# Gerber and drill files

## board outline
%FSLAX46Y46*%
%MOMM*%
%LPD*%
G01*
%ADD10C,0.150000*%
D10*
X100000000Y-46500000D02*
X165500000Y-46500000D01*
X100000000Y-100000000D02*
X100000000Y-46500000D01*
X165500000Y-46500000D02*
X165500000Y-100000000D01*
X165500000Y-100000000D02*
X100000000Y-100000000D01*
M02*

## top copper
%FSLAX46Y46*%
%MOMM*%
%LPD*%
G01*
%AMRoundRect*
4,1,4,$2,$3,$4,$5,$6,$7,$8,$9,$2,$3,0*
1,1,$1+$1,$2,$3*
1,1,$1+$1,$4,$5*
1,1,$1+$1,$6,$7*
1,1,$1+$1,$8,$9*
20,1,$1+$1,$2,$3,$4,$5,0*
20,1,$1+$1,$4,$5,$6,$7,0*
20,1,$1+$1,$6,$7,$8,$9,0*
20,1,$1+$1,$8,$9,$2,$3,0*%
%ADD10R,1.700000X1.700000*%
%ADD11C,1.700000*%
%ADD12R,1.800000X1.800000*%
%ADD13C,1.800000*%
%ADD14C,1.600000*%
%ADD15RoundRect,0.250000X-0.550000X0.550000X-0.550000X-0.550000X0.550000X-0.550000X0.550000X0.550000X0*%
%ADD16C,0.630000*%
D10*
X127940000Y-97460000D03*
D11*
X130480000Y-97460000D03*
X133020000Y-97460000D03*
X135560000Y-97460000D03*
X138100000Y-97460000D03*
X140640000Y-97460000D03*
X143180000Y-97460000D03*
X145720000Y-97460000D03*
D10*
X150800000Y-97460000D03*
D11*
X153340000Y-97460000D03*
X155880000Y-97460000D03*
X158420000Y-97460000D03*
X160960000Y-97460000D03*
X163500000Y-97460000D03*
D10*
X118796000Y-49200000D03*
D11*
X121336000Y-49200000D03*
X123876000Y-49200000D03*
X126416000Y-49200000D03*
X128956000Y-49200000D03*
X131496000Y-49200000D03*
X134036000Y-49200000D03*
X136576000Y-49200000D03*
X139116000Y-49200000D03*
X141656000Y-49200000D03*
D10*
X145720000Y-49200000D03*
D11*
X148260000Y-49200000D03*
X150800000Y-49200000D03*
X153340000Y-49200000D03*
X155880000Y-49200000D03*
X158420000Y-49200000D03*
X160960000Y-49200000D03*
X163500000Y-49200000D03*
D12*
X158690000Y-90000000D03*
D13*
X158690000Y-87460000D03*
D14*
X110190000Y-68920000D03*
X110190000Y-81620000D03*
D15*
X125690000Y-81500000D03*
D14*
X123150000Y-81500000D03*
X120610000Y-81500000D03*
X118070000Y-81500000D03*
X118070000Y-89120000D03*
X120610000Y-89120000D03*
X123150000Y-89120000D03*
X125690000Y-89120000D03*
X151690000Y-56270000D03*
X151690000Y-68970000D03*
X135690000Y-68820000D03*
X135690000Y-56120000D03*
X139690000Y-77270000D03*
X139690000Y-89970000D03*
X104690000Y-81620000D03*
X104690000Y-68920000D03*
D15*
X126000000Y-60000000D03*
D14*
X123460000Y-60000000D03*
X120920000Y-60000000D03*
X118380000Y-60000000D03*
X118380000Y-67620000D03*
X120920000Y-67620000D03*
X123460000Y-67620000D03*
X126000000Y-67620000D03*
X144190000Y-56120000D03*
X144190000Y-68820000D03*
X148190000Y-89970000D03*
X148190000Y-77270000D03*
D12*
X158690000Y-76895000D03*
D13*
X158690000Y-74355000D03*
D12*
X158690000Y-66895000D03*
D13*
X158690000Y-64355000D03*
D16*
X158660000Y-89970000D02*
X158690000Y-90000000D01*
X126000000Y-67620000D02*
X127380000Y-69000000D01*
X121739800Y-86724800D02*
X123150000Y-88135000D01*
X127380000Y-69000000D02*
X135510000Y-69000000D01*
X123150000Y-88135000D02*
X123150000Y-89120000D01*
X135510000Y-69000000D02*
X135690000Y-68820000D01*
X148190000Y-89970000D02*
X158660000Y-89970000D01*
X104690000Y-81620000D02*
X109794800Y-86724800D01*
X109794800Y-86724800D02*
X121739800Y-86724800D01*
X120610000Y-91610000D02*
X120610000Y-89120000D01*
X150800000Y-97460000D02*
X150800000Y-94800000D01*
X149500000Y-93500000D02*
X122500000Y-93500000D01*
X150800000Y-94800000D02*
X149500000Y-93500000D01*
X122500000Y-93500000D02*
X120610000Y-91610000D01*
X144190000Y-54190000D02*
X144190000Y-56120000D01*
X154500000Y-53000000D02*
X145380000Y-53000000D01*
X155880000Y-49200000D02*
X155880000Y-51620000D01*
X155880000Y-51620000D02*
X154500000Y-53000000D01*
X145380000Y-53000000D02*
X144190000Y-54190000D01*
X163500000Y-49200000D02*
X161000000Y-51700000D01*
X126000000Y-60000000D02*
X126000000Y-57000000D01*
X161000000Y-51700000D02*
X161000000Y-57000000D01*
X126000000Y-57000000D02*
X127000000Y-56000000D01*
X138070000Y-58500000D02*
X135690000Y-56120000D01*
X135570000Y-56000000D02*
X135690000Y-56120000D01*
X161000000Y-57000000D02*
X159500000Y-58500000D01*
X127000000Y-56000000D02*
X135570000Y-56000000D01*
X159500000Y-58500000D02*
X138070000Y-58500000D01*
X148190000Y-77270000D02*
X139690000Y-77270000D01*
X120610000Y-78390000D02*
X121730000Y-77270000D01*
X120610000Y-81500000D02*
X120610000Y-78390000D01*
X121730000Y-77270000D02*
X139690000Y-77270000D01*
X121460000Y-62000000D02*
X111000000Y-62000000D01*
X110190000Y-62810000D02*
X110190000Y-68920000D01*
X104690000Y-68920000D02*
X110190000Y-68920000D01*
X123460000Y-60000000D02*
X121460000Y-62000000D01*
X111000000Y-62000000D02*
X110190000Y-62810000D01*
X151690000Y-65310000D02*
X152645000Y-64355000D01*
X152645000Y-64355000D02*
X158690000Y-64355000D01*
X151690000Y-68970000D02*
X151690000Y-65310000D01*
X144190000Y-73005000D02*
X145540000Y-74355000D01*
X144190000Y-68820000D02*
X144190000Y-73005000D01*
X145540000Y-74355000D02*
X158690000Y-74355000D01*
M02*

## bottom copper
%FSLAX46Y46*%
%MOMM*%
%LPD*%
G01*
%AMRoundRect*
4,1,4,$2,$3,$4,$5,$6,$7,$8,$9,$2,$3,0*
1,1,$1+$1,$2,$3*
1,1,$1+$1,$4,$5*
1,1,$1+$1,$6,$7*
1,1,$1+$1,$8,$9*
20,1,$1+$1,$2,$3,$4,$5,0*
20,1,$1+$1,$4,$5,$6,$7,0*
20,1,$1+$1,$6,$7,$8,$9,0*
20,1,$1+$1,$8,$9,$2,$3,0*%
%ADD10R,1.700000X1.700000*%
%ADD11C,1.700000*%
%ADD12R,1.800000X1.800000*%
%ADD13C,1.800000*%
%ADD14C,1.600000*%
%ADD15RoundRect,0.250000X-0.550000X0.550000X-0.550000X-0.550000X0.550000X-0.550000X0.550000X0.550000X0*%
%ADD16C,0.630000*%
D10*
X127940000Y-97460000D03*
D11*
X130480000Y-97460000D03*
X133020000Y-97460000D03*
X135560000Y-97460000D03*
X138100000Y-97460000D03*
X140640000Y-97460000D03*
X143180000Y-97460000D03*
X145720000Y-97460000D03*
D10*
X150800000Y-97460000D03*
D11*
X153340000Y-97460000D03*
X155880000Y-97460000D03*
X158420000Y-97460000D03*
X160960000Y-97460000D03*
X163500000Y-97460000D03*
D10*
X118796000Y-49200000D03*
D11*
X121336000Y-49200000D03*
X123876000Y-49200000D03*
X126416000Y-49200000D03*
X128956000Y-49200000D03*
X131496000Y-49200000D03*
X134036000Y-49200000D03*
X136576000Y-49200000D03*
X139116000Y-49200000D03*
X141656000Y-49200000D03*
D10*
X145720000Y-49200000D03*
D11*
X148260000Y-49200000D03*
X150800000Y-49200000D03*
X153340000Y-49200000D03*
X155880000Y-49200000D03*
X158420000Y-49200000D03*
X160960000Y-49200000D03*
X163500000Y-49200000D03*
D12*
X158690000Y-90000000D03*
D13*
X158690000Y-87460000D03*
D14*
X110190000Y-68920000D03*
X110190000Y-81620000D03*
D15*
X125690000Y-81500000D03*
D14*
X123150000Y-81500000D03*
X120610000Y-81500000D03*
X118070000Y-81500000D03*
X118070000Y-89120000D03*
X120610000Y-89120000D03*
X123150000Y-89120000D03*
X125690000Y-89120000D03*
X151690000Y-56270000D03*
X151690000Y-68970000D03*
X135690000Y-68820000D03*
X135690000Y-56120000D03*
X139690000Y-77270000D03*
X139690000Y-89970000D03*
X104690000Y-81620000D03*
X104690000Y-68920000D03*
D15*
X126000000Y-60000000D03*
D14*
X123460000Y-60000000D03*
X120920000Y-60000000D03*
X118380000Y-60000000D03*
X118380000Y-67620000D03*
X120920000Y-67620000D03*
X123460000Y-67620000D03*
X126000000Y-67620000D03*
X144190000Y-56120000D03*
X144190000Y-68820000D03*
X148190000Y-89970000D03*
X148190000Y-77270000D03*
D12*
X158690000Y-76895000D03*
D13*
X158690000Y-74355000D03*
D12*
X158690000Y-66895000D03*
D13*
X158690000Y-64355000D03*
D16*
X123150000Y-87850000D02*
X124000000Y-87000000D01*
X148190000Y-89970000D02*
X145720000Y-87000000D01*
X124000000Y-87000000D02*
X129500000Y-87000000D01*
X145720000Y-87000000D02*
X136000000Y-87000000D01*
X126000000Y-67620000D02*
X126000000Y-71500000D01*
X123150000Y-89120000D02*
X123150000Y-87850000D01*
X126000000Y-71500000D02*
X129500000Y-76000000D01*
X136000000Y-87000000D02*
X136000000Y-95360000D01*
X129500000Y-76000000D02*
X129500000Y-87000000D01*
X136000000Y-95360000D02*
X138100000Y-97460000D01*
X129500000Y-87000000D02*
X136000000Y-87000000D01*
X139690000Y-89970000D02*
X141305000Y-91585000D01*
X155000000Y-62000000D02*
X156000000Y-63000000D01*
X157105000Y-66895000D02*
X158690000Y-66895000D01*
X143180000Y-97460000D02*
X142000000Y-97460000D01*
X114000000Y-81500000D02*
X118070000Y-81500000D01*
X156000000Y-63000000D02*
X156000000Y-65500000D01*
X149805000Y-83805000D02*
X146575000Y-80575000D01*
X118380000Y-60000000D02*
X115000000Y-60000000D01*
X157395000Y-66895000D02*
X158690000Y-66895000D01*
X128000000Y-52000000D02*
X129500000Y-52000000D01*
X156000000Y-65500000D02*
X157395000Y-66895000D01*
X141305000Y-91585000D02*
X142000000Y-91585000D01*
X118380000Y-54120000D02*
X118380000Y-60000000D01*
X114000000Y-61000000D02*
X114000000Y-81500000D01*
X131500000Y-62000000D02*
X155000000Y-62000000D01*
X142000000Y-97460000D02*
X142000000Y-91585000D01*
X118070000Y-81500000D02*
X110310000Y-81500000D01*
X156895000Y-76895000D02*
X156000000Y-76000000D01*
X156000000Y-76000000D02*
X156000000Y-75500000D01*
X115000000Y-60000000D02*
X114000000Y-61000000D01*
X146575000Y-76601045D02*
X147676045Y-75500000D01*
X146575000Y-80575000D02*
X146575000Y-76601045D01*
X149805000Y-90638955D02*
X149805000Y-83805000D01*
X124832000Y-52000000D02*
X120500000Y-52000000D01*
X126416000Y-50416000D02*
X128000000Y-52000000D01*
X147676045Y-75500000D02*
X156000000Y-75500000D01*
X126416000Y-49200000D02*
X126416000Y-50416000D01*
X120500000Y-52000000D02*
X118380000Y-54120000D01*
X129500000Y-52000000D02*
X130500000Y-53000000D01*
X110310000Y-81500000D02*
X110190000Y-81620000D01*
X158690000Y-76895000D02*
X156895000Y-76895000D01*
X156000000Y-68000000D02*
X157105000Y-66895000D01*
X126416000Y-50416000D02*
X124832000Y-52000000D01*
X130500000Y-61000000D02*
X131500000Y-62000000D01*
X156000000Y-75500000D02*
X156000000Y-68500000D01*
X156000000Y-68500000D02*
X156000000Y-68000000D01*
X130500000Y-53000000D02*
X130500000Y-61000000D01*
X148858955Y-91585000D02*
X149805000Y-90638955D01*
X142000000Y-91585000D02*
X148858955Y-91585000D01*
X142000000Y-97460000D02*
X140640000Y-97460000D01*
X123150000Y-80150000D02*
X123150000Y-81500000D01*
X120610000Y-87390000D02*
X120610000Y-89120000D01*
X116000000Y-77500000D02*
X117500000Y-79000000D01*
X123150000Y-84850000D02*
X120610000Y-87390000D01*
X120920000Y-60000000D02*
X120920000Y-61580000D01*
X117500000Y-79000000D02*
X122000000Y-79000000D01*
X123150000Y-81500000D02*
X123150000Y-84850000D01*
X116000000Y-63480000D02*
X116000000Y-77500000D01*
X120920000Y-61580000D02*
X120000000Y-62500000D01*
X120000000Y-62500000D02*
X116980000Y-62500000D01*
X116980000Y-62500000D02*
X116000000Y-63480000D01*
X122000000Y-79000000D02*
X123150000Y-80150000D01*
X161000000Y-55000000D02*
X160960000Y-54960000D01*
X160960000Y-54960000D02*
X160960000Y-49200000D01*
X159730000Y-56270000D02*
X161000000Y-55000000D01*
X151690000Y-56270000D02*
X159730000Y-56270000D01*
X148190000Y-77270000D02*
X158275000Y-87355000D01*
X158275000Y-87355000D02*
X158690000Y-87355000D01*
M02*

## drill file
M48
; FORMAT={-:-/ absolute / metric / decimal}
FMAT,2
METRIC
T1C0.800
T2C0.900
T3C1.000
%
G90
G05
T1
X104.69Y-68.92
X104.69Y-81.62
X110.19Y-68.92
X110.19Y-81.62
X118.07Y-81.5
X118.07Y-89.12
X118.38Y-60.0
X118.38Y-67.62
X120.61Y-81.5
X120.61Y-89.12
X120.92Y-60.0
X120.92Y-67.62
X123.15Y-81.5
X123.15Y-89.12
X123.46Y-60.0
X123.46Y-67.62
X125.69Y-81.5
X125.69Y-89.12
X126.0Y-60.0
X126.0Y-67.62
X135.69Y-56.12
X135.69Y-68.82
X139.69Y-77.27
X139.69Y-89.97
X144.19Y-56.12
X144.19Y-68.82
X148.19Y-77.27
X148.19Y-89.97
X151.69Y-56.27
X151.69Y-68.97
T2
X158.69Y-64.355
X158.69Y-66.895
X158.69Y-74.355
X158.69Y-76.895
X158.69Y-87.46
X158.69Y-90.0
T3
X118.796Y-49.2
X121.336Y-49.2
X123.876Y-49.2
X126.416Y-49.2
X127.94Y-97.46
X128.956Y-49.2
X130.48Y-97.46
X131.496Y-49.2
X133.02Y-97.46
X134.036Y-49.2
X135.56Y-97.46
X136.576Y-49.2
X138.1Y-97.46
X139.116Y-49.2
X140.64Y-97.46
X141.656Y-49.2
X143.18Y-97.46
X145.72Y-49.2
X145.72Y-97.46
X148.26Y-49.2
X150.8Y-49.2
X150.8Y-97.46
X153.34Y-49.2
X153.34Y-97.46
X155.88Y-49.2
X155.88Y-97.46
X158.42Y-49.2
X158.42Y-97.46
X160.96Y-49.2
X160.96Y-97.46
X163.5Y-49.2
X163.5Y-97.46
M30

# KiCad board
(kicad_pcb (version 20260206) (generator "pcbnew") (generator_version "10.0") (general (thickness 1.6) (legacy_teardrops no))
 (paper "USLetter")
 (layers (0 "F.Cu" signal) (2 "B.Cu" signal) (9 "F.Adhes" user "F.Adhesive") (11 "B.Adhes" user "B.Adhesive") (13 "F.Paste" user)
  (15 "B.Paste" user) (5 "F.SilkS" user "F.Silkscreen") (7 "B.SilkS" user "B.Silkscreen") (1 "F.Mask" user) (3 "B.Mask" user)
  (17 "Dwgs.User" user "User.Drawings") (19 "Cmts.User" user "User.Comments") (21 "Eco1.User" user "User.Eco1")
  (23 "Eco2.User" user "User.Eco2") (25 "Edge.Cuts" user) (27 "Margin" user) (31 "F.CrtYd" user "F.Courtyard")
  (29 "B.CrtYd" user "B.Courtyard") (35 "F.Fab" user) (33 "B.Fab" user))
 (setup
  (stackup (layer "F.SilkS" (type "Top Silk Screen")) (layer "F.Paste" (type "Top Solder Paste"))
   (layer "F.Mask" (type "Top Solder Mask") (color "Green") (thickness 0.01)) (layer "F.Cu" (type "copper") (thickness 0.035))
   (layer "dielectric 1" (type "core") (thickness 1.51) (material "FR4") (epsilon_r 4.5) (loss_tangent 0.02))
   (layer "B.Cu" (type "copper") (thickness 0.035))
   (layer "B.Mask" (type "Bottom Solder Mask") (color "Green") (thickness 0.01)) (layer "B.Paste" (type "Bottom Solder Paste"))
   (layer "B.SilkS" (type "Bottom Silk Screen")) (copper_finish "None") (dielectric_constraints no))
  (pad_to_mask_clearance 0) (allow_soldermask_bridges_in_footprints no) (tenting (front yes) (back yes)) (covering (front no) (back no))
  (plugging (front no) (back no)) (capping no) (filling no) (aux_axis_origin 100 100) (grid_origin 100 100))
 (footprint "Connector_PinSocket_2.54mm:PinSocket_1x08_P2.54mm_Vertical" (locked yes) (layer "F.Cu") (at 127.94 97.46 90)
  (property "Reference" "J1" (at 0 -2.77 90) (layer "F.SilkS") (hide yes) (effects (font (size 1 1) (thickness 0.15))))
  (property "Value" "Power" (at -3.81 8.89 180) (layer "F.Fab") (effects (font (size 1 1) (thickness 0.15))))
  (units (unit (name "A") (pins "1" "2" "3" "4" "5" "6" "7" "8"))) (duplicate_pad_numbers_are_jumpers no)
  (pad "1" thru_hole rect (at 0 0 90) (size 1.7 1.7) (drill 1) (layers "*.Cu" "*.Mask") (remove_unused_layers no)
   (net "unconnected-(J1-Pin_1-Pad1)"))
  (pad "2" thru_hole circle (at 0 2.54 90) (size 1.7 1.7) (drill 1) (layers "*.Cu" "*.Mask") (remove_unused_layers no) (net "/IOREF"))
  (pad "3" thru_hole circle (at 0 5.08 90) (size 1.7 1.7) (drill 1) (layers "*.Cu" "*.Mask") (remove_unused_layers no) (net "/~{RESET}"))
  (pad "4" thru_hole circle (at 0 7.62 90) (size 1.7 1.7) (drill 1) (layers "*.Cu" "*.Mask") (remove_unused_layers no) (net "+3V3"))
  (pad "5" thru_hole circle (at 0 10.16 90) (size 1.7 1.7) (drill 1) (layers "*.Cu" "*.Mask") (remove_unused_layers no) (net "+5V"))
  (pad "6" thru_hole circle (at 0 12.7 90) (size 1.7 1.7) (drill 1) (layers "*.Cu" "*.Mask") (remove_unused_layers no) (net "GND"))
  (pad "7" thru_hole circle (at 0 15.24 90) (size 1.7 1.7) (drill 1) (layers "*.Cu" "*.Mask") (remove_unused_layers no) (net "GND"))
  (pad "8" thru_hole circle (at 0 17.78 90) (size 1.7 1.7) (drill 1) (layers "*.Cu" "*.Mask") (remove_unused_layers no) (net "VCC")))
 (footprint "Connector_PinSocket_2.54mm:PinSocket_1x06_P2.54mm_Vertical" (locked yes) (layer "F.Cu") (at 150.8 97.46 90)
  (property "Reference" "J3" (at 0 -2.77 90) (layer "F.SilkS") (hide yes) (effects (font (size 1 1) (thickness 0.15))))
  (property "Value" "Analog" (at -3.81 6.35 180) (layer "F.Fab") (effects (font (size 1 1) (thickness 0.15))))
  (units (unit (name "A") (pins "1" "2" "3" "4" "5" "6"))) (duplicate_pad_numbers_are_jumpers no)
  (pad "1" thru_hole rect (at 0 0 90) (size 1.7 1.7) (drill 1) (layers "*.Cu" "*.Mask") (remove_unused_layers no) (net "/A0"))
  (pad "2" thru_hole circle (at 0 2.54 90) (size 1.7 1.7) (drill 1) (layers "*.Cu" "*.Mask") (remove_unused_layers no) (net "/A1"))
  (pad "3" thru_hole circle (at 0 5.08 90) (size 1.7 1.7) (drill 1) (layers "*.Cu" "*.Mask") (remove_unused_layers no) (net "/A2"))
  (pad "4" thru_hole circle (at 0 7.62 90) (size 1.7 1.7) (drill 1) (layers "*.Cu" "*.Mask") (remove_unused_layers no) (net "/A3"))
  (pad "5" thru_hole circle (at 0 10.16 90) (size 1.7 1.7) (drill 1) (layers "*.Cu" "*.Mask") (remove_unused_layers no) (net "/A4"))
  (pad "6" thru_hole circle (at 0 12.7 90) (size 1.7 1.7) (drill 1) (layers "*.Cu" "*.Mask") (remove_unused_layers no) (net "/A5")))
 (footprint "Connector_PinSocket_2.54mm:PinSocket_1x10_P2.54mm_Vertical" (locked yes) (layer "F.Cu") (at 118.796 49.2 90)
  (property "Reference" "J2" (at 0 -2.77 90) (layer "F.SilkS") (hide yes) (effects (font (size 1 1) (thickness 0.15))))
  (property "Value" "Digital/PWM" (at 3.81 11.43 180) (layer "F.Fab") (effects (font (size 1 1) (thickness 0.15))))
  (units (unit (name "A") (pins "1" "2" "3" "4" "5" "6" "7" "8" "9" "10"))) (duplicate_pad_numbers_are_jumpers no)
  (pad "1" thru_hole rect (at 0 0 90) (size 1.7 1.7) (drill 1) (layers "*.Cu" "*.Mask") (remove_unused_layers no) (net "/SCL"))
  (pad "2" thru_hole circle (at 0 2.54 90) (size 1.7 1.7) (drill 1) (layers "*.Cu" "*.Mask") (remove_unused_layers no) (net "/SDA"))
  (pad "3" thru_hole circle (at 0 5.08 90) (size 1.7 1.7) (drill 1) (layers "*.Cu" "*.Mask") (remove_unused_layers no) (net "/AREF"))
  (pad "4" thru_hole circle (at 0 7.62 90) (size 1.7 1.7) (drill 1) (layers "*.Cu" "*.Mask") (remove_unused_layers no) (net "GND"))
  (pad "5" thru_hole circle (at 0 10.16 90) (size 1.7 1.7) (drill 1) (layers "*.Cu" "*.Mask") (remove_unused_layers no) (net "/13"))
  (pad "6" thru_hole circle (at 0 12.7 90) (size 1.7 1.7) (drill 1) (layers "*.Cu" "*.Mask") (remove_unused_layers no) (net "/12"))
  (pad "7" thru_hole circle (at 0 15.24 90) (size 1.7 1.7) (drill 1) (layers "*.Cu" "*.Mask") (remove_unused_layers no) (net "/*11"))
  (pad "8" thru_hole circle (at 0 17.78 90) (size 1.7 1.7) (drill 1) (layers "*.Cu" "*.Mask") (remove_unused_layers no) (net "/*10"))
  (pad "9" thru_hole circle (at 0 20.32 90) (size 1.7 1.7) (drill 1) (layers "*.Cu" "*.Mask") (remove_unused_layers no) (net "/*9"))
  (pad "10" thru_hole circle (at 0 22.86 90) (size 1.7 1.7) (drill 1) (layers "*.Cu" "*.Mask") (remove_unused_layers no) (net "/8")))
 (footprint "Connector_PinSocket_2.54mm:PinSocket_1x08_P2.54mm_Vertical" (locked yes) (layer "F.Cu") (at 145.72 49.2 90)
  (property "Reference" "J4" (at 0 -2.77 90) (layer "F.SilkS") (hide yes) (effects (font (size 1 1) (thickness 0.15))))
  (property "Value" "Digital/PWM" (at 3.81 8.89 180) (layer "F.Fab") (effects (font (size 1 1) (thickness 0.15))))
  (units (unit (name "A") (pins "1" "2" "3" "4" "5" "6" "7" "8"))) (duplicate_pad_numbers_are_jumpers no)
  (pad "1" thru_hole rect (at 0 0 90) (size 1.7 1.7) (drill 1) (layers "*.Cu" "*.Mask") (remove_unused_layers no) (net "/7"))
  (pad "2" thru_hole circle (at 0 2.54 90) (size 1.7 1.7) (drill 1) (layers "*.Cu" "*.Mask") (remove_unused_layers no) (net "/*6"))
  (pad "3" thru_hole circle (at 0 5.08 90) (size 1.7 1.7) (drill 1) (layers "*.Cu" "*.Mask") (remove_unused_layers no) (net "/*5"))
  (pad "4" thru_hole circle (at 0 7.62 90) (size 1.7 1.7) (drill 1) (layers "*.Cu" "*.Mask") (remove_unused_layers no) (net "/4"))
  (pad "5" thru_hole circle (at 0 10.16 90) (size 1.7 1.7) (drill 1) (layers "*.Cu" "*.Mask") (remove_unused_layers no) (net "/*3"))
  (pad "6" thru_hole circle (at 0 12.7 90) (size 1.7 1.7) (drill 1) (layers "*.Cu" "*.Mask") (remove_unused_layers no) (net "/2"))
  (pad "7" thru_hole circle (at 0 15.24 90) (size 1.7 1.7) (drill 1) (layers "*.Cu" "*.Mask") (remove_unused_layers no) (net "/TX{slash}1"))
  (pad "8" thru_hole circle (at 0 17.78 90) (size 1.7 1.7) (drill 1) (layers "*.Cu" "*.Mask") (remove_unused_layers no) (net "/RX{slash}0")))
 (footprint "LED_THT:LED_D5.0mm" (layer "F.Cu") (at 158.69 90 90)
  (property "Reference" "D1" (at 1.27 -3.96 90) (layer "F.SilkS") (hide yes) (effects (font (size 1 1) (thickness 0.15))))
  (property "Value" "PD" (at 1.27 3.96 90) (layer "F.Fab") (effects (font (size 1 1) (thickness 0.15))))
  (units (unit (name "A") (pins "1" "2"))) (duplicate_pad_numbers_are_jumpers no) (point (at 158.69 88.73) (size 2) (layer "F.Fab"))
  (pad "1" thru_hole rect (at 0 0 90) (size 1.8 1.8) (drill 0.9) (layers "*.Cu" "*.Mask") (remove_unused_layers no) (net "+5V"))
  (pad "2" thru_hole circle (at 2.54 0 90) (size 1.8 1.8) (drill 0.9) (layers "*.Cu" "*.Mask") (remove_unused_layers no) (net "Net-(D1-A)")))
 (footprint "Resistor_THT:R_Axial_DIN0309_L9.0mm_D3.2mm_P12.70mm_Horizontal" (layer "F.Cu") (at 110.19 68.92 -90)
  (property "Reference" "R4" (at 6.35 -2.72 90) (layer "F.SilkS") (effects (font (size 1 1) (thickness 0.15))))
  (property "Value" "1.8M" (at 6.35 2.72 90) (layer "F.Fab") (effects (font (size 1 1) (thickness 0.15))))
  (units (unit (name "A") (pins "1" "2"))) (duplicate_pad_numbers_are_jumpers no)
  (pad "1" thru_hole circle (at 0 0 270) (size 1.6 1.6) (drill 0.8) (layers "*.Cu" "*.Mask") (remove_unused_layers no) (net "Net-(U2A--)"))
  (pad "2" thru_hole circle (at 12.7 0 270) (size 1.6 1.6) (drill 0.8) (layers "*.Cu" "*.Mask") (remove_unused_layers no) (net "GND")))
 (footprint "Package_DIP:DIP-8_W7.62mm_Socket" (layer "F.Cu") (at 125.69 81.5 -90)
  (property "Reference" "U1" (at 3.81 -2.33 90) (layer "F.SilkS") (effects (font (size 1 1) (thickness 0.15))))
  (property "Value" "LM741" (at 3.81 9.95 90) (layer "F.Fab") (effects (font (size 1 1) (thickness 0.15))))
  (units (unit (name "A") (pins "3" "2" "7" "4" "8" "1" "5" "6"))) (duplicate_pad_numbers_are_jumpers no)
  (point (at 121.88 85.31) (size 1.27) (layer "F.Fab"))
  (pad "1" thru_hole roundrect (at 0 0 270) (size 1.6 1.6) (drill 0.8) (layers "*.Cu" "*.Mask") (remove_unused_layers no)
   (roundrect_rratio 0.15625) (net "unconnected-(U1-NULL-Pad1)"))
  (pad "2" thru_hole circle (at 0 2.54 270) (size 1.6 1.6) (drill 0.8) (layers "*.Cu" "*.Mask") (remove_unused_layers no) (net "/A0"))
  (pad "3" thru_hole circle (at 0 5.08 270) (size 1.6 1.6) (drill 0.8) (layers "*.Cu" "*.Mask") (remove_unused_layers no) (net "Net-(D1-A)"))
  (pad "4" thru_hole circle (at 0 7.62 270) (size 1.6 1.6) (drill 0.8) (layers "*.Cu" "*.Mask") (remove_unused_layers no) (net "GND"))
  (pad "5" thru_hole circle (at 7.62 7.62 270) (size 1.6 1.6) (drill 0.8) (layers "*.Cu" "*.Mask") (remove_unused_layers no)
   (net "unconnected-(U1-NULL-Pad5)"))
  (pad "6" thru_hole circle (at 7.62 5.08 270) (size 1.6 1.6) (drill 0.8) (layers "*.Cu" "*.Mask") (remove_unused_layers no) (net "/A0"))
  (pad "7" thru_hole circle (at 7.62 2.54 270) (size 1.6 1.6) (drill 0.8) (layers "*.Cu" "*.Mask") (remove_unused_layers no) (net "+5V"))
  (pad "8" thru_hole circle (at 7.62 0 270) (size 1.6 1.6) (drill 0.8) (layers "*.Cu" "*.Mask") (remove_unused_layers no)
   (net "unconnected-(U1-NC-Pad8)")))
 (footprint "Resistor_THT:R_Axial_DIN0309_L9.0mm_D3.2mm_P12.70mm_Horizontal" (layer "F.Cu") (at 151.69 56.27 -90)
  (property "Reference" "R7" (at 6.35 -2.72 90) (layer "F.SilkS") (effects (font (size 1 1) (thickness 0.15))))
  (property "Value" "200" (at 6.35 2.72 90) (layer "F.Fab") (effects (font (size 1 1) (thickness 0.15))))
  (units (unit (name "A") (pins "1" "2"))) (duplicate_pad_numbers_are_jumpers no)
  (pad "1" thru_hole circle (at 0 0 270) (size 1.6 1.6) (drill 0.8) (layers "*.Cu" "*.Mask") (remove_unused_layers no) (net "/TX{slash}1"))
  (pad "2" thru_hole circle (at 12.7 0 270) (size 1.6 1.6) (drill 0.8) (layers "*.Cu" "*.Mask") (remove_unused_layers no) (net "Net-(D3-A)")))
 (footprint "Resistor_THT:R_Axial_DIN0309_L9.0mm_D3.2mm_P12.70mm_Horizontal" (layer "F.Cu") (at 135.69 68.82 90)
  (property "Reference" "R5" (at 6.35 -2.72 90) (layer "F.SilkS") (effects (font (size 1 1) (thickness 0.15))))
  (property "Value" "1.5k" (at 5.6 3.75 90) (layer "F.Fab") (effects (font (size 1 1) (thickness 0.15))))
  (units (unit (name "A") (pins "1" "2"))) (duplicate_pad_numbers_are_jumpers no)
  (pad "1" thru_hole circle (at 0 0 90) (size 1.6 1.6) (drill 0.8) (layers "*.Cu" "*.Mask") (remove_unused_layers no) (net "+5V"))
  (pad "2" thru_hole circle (at 12.7 0 90) (size 1.6 1.6) (drill 0.8) (layers "*.Cu" "*.Mask") (remove_unused_layers no) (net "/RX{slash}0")))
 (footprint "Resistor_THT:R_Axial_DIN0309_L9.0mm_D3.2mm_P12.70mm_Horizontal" (layer "F.Cu") (at 139.69 77.27 -90)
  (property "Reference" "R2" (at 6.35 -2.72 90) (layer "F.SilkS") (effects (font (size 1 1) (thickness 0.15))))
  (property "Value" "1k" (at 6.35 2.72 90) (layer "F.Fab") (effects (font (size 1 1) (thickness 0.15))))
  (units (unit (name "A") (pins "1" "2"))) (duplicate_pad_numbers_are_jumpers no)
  (pad "1" thru_hole circle (at 0 0 270) (size 1.6 1.6) (drill 0.8) (layers "*.Cu" "*.Mask") (remove_unused_layers no) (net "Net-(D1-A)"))
  (pad "2" thru_hole circle (at 12.7 0 270) (size 1.6 1.6) (drill 0.8) (layers "*.Cu" "*.Mask") (remove_unused_layers no) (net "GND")))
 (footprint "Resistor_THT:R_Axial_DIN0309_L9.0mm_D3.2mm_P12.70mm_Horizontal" (layer "F.Cu") (at 104.69 81.62 90)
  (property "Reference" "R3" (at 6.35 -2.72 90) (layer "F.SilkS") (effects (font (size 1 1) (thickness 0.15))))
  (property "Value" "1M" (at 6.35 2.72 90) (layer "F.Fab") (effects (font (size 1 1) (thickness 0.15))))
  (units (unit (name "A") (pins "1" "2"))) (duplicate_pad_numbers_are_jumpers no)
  (pad "1" thru_hole circle (at 0 0 90) (size 1.6 1.6) (drill 0.8) (layers "*.Cu" "*.Mask") (remove_unused_layers no) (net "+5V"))
  (pad "2" thru_hole circle (at 12.7 0 90) (size 1.6 1.6) (drill 0.8) (layers "*.Cu" "*.Mask") (remove_unused_layers no) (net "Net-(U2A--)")))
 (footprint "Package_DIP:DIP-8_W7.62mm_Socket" (layer "F.Cu") (at 126 60 -90)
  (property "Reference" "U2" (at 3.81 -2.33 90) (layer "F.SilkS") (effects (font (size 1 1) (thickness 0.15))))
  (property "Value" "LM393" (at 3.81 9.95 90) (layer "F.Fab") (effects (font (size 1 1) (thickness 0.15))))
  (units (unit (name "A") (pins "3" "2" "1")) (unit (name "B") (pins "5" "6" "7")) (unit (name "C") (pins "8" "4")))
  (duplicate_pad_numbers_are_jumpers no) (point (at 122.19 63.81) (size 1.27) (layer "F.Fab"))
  (pad "1" thru_hole roundrect (at 0 0 270) (size 1.6 1.6) (drill 0.8) (layers "*.Cu" "*.Mask") (remove_unused_layers no)
   (roundrect_rratio 0.15625) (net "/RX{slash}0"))
  (pad "2" thru_hole circle (at 0 2.54 270) (size 1.6 1.6) (drill 0.8) (layers "*.Cu" "*.Mask") (remove_unused_layers no)
   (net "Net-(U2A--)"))
  (pad "3" thru_hole circle (at 0 5.08 270) (size 1.6 1.6) (drill 0.8) (layers "*.Cu" "*.Mask") (remove_unused_layers no) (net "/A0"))
  (pad "4" thru_hole circle (at 0 7.62 270) (size 1.6 1.6) (drill 0.8) (layers "*.Cu" "*.Mask") (remove_unused_layers no) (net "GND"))
  (pad "5" thru_hole circle (at 7.62 7.62 270) (size 1.6 1.6) (drill 0.8) (layers "*.Cu" "*.Mask") (remove_unused_layers no)
   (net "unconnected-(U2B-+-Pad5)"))
  (pad "6" thru_hole circle (at 7.62 5.08 270) (size 1.6 1.6) (drill 0.8) (layers "*.Cu" "*.Mask") (remove_unused_layers no)
   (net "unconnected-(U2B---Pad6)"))
  (pad "7" thru_hole circle (at 7.62 2.54 270) (size 1.6 1.6) (drill 0.8) (layers "*.Cu" "*.Mask") (remove_unused_layers no)
   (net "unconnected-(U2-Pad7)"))
  (pad "8" thru_hole circle (at 7.62 0 270) (size 1.6 1.6) (drill 0.8) (layers "*.Cu" "*.Mask") (remove_unused_layers no) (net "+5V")))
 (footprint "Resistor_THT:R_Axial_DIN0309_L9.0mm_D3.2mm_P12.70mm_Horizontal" (layer "F.Cu") (at 144.19 56.12 -90)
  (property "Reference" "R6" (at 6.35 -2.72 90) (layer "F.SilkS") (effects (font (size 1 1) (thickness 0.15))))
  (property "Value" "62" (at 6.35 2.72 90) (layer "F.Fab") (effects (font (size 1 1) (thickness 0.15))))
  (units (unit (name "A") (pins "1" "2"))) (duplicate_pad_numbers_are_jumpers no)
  (pad "1" thru_hole circle (at 0 0 270) (size 1.6 1.6) (drill 0.8) (layers "*.Cu" "*.Mask") (remove_unused_layers no) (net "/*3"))
  (pad "2" thru_hole circle (at 12.7 0 270) (size 1.6 1.6) (drill 0.8) (layers "*.Cu" "*.Mask") (remove_unused_layers no) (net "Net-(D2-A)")))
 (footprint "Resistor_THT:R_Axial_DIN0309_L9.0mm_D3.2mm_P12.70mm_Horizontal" (layer "F.Cu") (at 148.19 89.97 90)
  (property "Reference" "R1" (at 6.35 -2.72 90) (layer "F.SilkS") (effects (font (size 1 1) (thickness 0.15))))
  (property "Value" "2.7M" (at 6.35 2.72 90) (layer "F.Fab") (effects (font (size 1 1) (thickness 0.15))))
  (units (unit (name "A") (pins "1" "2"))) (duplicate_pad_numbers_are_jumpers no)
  (pad "1" thru_hole circle (at 0 0 90) (size 1.6 1.6) (drill 0.8) (layers "*.Cu" "*.Mask") (remove_unused_layers no) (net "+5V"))
  (pad "2" thru_hole circle (at 12.7 0 90) (size 1.6 1.6) (drill 0.8) (layers "*.Cu" "*.Mask") (remove_unused_layers no) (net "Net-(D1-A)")))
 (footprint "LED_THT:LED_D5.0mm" (layer "F.Cu") (at 158.69 76.895 90)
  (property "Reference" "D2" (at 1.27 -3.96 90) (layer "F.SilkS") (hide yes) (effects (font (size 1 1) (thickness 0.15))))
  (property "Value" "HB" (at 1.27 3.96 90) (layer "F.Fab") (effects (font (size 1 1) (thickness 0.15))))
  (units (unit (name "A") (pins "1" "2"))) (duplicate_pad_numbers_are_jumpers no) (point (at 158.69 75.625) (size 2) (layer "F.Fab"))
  (pad "1" thru_hole rect (at 0 0 90) (size 1.8 1.8) (drill 0.9) (layers "*.Cu" "*.Mask") (remove_unused_layers no) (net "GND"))
  (pad "2" thru_hole circle (at 2.54 0 90) (size 1.8 1.8) (drill 0.9) (layers "*.Cu" "*.Mask") (remove_unused_layers no) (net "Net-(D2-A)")))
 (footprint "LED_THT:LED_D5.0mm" (layer "F.Cu") (at 158.69 66.895 90)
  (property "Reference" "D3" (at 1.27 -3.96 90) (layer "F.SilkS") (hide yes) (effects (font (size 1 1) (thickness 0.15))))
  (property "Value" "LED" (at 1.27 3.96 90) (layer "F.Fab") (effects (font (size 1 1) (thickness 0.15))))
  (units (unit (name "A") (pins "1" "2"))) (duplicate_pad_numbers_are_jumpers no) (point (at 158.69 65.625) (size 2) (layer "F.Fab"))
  (pad "1" thru_hole rect (at 0 0 90) (size 1.8 1.8) (drill 0.9) (layers "*.Cu" "*.Mask") (remove_unused_layers no) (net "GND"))
  (pad "2" thru_hole circle (at 2.54 0 90) (size 1.8 1.8) (drill 0.9) (layers "*.Cu" "*.Mask") (remove_unused_layers no) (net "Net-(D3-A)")))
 (gr_line (start 100 46.5) (end 165.5 46.5) (stroke (width 0.15) (type default)) (layer "Edge.Cuts"))
 (gr_line (start 100 100) (end 100 46.5) (stroke (width 0.15) (type default)) (layer "Edge.Cuts"))
 (gr_line (start 165.5 46.5) (end 165.5 100) (stroke (width 0.15) (type default)) (layer "Edge.Cuts"))
 (gr_line (start 165.5 100) (end 100 100) (stroke (width 0.15) (type default)) (layer "Edge.Cuts"))
 (segment (start 158.66 89.97) (end 158.69 90) (width 0.63) (layer "F.Cu") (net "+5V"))
 (segment (start 126 67.62) (end 127.38 69) (width 0.63) (layer "F.Cu") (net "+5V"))
 (segment (start 121.7398 86.7248) (end 123.15 88.135) (width 0.63) (layer "F.Cu") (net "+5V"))
 (segment (start 127.38 69) (end 135.51 69) (width 0.63) (layer "F.Cu") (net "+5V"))
 (segment (start 123.15 88.135) (end 123.15 89.12) (width 0.63) (layer "F.Cu") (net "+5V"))
 (segment (start 135.51 69) (end 135.69 68.82) (width 0.63) (layer "F.Cu") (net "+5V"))
 (segment (start 148.19 89.97) (end 158.66 89.97) (width 0.63) (layer "F.Cu") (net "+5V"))
 (segment (start 104.69 81.62) (end 109.7948 86.7248) (width 0.63) (layer "F.Cu") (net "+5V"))
 (segment (start 109.7948 86.7248) (end 121.7398 86.7248) (width 0.63) (layer "F.Cu") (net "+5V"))
 (segment (start 123.15 87.85) (end 124 87) (width 0.63) (layer "B.Cu") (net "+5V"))
 (segment (start 148.19 89.97) (end 145.72 87) (width 0.63) (layer "B.Cu") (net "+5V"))
 (segment (start 124 87) (end 129.5 87) (width 0.63) (layer "B.Cu") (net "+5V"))
 (segment (start 145.72 87) (end 136 87) (width 0.63) (layer "B.Cu") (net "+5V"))
 (segment (start 126 67.62) (end 126 71.5) (width 0.63) (layer "B.Cu") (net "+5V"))
 (segment (start 123.15 89.12) (end 123.15 87.85) (width 0.63) (layer "B.Cu") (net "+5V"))
 (segment (start 126 71.5) (end 129.5 76) (width 0.63) (layer "B.Cu") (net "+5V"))
 (segment (start 136 87) (end 136 95.36) (width 0.63) (layer "B.Cu") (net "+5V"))
 (segment (start 129.5 76) (end 129.5 87) (width 0.63) (layer "B.Cu") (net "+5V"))
 (segment (start 136 95.36) (end 138.1 97.46) (width 0.63) (layer "B.Cu") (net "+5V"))
 (segment (start 129.5 87) (end 136 87) (width 0.63) (layer "B.Cu") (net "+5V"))
 (segment (start 139.69 89.97) (end 141.305 91.585) (width 0.63) (layer "B.Cu") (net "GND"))
 (segment (start 155 62) (end 156 63) (width 0.63) (layer "B.Cu") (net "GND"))
 (segment (start 157.105 66.895) (end 158.69 66.895) (width 0.63) (layer "B.Cu") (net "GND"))
 (segment (start 143.18 97.46) (end 142 97.46) (width 0.63) (layer "B.Cu") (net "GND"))
 (segment (start 114 81.5) (end 118.07 81.5) (width 0.63) (layer "B.Cu") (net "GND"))
 (segment (start 156 63) (end 156 65.5) (width 0.63) (layer "B.Cu") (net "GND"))
 (segment (start 149.805 83.805) (end 146.575 80.575) (width 0.63) (layer "B.Cu") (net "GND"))
 (segment (start 118.38 60) (end 115 60) (width 0.63) (layer "B.Cu") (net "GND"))
 (segment (start 157.395 66.895) (end 158.69 66.895) (width 0.63) (layer "B.Cu") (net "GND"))
 (segment (start 128 52) (end 129.5 52) (width 0.63) (layer "B.Cu") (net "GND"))
 (segment (start 156 65.5) (end 157.395 66.895) (width 0.63) (layer "B.Cu") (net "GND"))
 (segment (start 141.305 91.585) (end 142 91.585) (width 0.63) (layer "B.Cu") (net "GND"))
 (segment (start 118.38 54.12) (end 118.38 60) (width 0.63) (layer "B.Cu") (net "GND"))
 (segment (start 114 61) (end 114 81.5) (width 0.63) (layer "B.Cu") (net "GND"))
 (segment (start 131.5 62) (end 155 62) (width 0.63) (layer "B.Cu") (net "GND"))
 (segment (start 142 97.46) (end 142 91.585) (width 0.63) (layer "B.Cu") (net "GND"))
 (segment (start 118.07 81.5) (end 110.31 81.5) (width 0.63) (layer "B.Cu") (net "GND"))
 (segment (start 156.895 76.895) (end 156 76) (width 0.63) (layer "B.Cu") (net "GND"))
 (segment (start 156 76) (end 156 75.5) (width 0.63) (layer "B.Cu") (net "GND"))
 (segment (start 115 60) (end 114 61) (width 0.63) (layer "B.Cu") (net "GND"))
 (segment (start 146.575 76.601045) (end 147.676045 75.5) (width 0.63) (layer "B.Cu") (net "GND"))
 (segment (start 146.575 80.575) (end 146.575 76.601045) (width 0.63) (layer "B.Cu") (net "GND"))
 (segment (start 149.805 90.638955) (end 149.805 83.805) (width 0.63) (layer "B.Cu") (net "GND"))
 (segment (start 124.832 52) (end 120.5 52) (width 0.63) (layer "B.Cu") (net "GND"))
 (segment (start 126.416 50.416) (end 128 52) (width 0.63) (layer "B.Cu") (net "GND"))
 (segment (start 147.676045 75.5) (end 156 75.5) (width 0.63) (layer "B.Cu") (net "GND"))
 (segment (start 126.416 49.2) (end 126.416 50.416) (width 0.63) (layer "B.Cu") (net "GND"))
 (segment (start 120.5 52) (end 118.38 54.12) (width 0.63) (layer "B.Cu") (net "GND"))
 (segment (start 129.5 52) (end 130.5 53) (width 0.63) (layer "B.Cu") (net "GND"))
 (segment (start 110.31 81.5) (end 110.19 81.62) (width 0.63) (layer "B.Cu") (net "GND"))
 (segment (start 158.69 76.895) (end 156.895 76.895) (width 0.63) (layer "B.Cu") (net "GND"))
 (segment (start 156 68) (end 157.105 66.895) (width 0.63) (layer "B.Cu") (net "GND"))
 (segment (start 126.416 50.416) (end 124.832 52) (width 0.63) (layer "B.Cu") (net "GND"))
 (segment (start 130.5 61) (end 131.5 62) (width 0.63) (layer "B.Cu") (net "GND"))
 (segment (start 156 75.5) (end 156 68.5) (width 0.63) (layer "B.Cu") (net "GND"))
 (segment (start 156 68.5) (end 156 68) (width 0.63) (layer "B.Cu") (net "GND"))
 (segment (start 130.5 53) (end 130.5 61) (width 0.63) (layer "B.Cu") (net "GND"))
 (segment (start 148.858955 91.585) (end 149.805 90.638955) (width 0.63) (layer "B.Cu") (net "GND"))
 (segment (start 142 91.585) (end 148.858955 91.585) (width 0.63) (layer "B.Cu") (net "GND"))
 (segment (start 142 97.46) (end 140.64 97.46) (width 0.63) (layer "B.Cu") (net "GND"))
 (segment (start 120.61 91.61) (end 120.61 89.12) (width 0.63) (layer "F.Cu") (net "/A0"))
 (segment (start 150.8 97.46) (end 150.8 94.8) (width 0.63) (layer "F.Cu") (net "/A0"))
 (segment (start 149.5 93.5) (end 122.5 93.5) (width 0.63) (layer "F.Cu") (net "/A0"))
 (segment (start 150.8 94.8) (end 149.5 93.5) (width 0.63) (layer "F.Cu") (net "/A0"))
 (segment (start 122.5 93.5) (end 120.61 91.61) (width 0.63) (layer "F.Cu") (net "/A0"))
 (segment (start 123.15 80.15) (end 123.15 81.5) (width 0.63) (layer "B.Cu") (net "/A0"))
 (segment (start 120.61 87.39) (end 120.61 89.12) (width 0.63) (layer "B.Cu") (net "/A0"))
 (segment (start 116 77.5) (end 117.5 79) (width 0.63) (layer "B.Cu") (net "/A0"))
 (segment (start 123.15 84.85) (end 120.61 87.39) (width 0.63) (layer "B.Cu") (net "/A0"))
 (segment (start 120.92 60) (end 120.92 61.58) (width 0.63) (layer "B.Cu") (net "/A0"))
 (segment (start 117.5 79) (end 122 79) (width 0.63) (layer "B.Cu") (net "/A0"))
 (segment (start 123.15 81.5) (end 123.15 84.85) (width 0.63) (layer "B.Cu") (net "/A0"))
 (segment (start 116 63.48) (end 116 77.5) (width 0.63) (layer "B.Cu") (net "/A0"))
 (segment (start 120.92 61.58) (end 120 62.5) (width 0.63) (layer "B.Cu") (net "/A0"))
 (segment (start 120 62.5) (end 116.98 62.5) (width 0.63) (layer "B.Cu") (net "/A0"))
 (segment (start 116.98 62.5) (end 116 63.48) (width 0.63) (layer "B.Cu") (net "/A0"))
 (segment (start 122 79) (end 123.15 80.15) (width 0.63) (layer "B.Cu") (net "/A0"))
 (segment (start 144.19 54.19) (end 144.19 56.12) (width 0.63) (layer "F.Cu") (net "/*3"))
 (segment (start 154.5 53) (end 145.38 53) (width 0.63) (layer "F.Cu") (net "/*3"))
 (segment (start 155.88 49.2) (end 155.88 51.62) (width 0.63) (layer "F.Cu") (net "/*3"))
 (segment (start 155.88 51.62) (end 154.5 53) (width 0.63) (layer "F.Cu") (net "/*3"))
 (segment (start 145.38 53) (end 144.19 54.19) (width 0.63) (layer "F.Cu") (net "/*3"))
 (segment (start 161 55) (end 160.96 54.96) (width 0.63) (layer "B.Cu") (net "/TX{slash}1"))
 (segment (start 160.96 54.96) (end 160.96 49.2) (width 0.63) (layer "B.Cu") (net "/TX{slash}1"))
 (segment (start 159.73 56.27) (end 161 55) (width 0.63) (layer "B.Cu") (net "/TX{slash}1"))
 (segment (start 151.69 56.27) (end 159.73 56.27) (width 0.63) (layer "B.Cu") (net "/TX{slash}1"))
 (segment (start 163.5 49.2) (end 161 51.7) (width 0.63) (layer "F.Cu") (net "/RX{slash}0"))
 (segment (start 126 60) (end 126 57) (width 0.63) (layer "F.Cu") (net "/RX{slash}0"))
 (segment (start 161 51.7) (end 161 57) (width 0.63) (layer "F.Cu") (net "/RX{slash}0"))
 (segment (start 126 57) (end 127 56) (width 0.63) (layer "F.Cu") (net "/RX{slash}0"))
 (segment (start 138.07 58.5) (end 135.69 56.12) (width 0.63) (layer "F.Cu") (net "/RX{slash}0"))
 (segment (start 135.57 56) (end 135.69 56.12) (width 0.63) (layer "F.Cu") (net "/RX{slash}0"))
 (segment (start 161 57) (end 159.5 58.5) (width 0.63) (layer "F.Cu") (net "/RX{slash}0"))
 (segment (start 127 56) (end 135.57 56) (width 0.63) (layer "F.Cu") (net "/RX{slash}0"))
 (segment (start 159.5 58.5) (end 138.07 58.5) (width 0.63) (layer "F.Cu") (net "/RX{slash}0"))
 (segment (start 148.19 77.27) (end 139.69 77.27) (width 0.63) (layer "F.Cu") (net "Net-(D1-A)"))
 (segment (start 120.61 78.39) (end 121.73 77.27) (width 0.63) (layer "F.Cu") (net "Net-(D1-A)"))
 (segment (start 120.61 81.5) (end 120.61 78.39) (width 0.63) (layer "F.Cu") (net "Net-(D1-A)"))
 (segment (start 121.73 77.27) (end 139.69 77.27) (width 0.63) (layer "F.Cu") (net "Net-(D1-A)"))
 (segment (start 148.19 77.27) (end 158.275 87.355) (width 0.63) (layer "B.Cu") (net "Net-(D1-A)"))
 (segment (start 158.275 87.355) (end 158.69 87.355) (width 0.63) (layer "B.Cu") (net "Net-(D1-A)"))
 (segment (start 121.46 62) (end 111 62) (width 0.63) (layer "F.Cu") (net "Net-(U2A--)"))
 (segment (start 110.19 62.81) (end 110.19 68.92) (width 0.63) (layer "F.Cu") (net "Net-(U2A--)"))
 (segment (start 104.69 68.92) (end 110.19 68.92) (width 0.63) (layer "F.Cu") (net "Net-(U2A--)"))
 (segment (start 123.46 60) (end 121.46 62) (width 0.63) (layer "F.Cu") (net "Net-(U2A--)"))
 (segment (start 111 62) (end 110.19 62.81) (width 0.63) (layer "F.Cu") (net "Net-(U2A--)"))
 (segment (start 151.69 65.31) (end 152.645 64.355) (width 0.63) (layer "F.Cu") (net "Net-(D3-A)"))
 (segment (start 152.645 64.355) (end 158.69 64.355) (width 0.63) (layer "F.Cu") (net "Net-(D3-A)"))
 (segment (start 151.69 68.97) (end 151.69 65.31) (width 0.63) (layer "F.Cu") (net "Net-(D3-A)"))
 (segment (start 144.19 73.005) (end 145.54 74.355) (width 0.63) (layer "F.Cu") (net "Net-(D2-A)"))
 (segment (start 144.19 68.82) (end 144.19 73.005) (width 0.63) (layer "F.Cu") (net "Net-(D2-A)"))
 (segment (start 145.54 74.355) (end 158.69 74.355) (width 0.63) (layer "F.Cu") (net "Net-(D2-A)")))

